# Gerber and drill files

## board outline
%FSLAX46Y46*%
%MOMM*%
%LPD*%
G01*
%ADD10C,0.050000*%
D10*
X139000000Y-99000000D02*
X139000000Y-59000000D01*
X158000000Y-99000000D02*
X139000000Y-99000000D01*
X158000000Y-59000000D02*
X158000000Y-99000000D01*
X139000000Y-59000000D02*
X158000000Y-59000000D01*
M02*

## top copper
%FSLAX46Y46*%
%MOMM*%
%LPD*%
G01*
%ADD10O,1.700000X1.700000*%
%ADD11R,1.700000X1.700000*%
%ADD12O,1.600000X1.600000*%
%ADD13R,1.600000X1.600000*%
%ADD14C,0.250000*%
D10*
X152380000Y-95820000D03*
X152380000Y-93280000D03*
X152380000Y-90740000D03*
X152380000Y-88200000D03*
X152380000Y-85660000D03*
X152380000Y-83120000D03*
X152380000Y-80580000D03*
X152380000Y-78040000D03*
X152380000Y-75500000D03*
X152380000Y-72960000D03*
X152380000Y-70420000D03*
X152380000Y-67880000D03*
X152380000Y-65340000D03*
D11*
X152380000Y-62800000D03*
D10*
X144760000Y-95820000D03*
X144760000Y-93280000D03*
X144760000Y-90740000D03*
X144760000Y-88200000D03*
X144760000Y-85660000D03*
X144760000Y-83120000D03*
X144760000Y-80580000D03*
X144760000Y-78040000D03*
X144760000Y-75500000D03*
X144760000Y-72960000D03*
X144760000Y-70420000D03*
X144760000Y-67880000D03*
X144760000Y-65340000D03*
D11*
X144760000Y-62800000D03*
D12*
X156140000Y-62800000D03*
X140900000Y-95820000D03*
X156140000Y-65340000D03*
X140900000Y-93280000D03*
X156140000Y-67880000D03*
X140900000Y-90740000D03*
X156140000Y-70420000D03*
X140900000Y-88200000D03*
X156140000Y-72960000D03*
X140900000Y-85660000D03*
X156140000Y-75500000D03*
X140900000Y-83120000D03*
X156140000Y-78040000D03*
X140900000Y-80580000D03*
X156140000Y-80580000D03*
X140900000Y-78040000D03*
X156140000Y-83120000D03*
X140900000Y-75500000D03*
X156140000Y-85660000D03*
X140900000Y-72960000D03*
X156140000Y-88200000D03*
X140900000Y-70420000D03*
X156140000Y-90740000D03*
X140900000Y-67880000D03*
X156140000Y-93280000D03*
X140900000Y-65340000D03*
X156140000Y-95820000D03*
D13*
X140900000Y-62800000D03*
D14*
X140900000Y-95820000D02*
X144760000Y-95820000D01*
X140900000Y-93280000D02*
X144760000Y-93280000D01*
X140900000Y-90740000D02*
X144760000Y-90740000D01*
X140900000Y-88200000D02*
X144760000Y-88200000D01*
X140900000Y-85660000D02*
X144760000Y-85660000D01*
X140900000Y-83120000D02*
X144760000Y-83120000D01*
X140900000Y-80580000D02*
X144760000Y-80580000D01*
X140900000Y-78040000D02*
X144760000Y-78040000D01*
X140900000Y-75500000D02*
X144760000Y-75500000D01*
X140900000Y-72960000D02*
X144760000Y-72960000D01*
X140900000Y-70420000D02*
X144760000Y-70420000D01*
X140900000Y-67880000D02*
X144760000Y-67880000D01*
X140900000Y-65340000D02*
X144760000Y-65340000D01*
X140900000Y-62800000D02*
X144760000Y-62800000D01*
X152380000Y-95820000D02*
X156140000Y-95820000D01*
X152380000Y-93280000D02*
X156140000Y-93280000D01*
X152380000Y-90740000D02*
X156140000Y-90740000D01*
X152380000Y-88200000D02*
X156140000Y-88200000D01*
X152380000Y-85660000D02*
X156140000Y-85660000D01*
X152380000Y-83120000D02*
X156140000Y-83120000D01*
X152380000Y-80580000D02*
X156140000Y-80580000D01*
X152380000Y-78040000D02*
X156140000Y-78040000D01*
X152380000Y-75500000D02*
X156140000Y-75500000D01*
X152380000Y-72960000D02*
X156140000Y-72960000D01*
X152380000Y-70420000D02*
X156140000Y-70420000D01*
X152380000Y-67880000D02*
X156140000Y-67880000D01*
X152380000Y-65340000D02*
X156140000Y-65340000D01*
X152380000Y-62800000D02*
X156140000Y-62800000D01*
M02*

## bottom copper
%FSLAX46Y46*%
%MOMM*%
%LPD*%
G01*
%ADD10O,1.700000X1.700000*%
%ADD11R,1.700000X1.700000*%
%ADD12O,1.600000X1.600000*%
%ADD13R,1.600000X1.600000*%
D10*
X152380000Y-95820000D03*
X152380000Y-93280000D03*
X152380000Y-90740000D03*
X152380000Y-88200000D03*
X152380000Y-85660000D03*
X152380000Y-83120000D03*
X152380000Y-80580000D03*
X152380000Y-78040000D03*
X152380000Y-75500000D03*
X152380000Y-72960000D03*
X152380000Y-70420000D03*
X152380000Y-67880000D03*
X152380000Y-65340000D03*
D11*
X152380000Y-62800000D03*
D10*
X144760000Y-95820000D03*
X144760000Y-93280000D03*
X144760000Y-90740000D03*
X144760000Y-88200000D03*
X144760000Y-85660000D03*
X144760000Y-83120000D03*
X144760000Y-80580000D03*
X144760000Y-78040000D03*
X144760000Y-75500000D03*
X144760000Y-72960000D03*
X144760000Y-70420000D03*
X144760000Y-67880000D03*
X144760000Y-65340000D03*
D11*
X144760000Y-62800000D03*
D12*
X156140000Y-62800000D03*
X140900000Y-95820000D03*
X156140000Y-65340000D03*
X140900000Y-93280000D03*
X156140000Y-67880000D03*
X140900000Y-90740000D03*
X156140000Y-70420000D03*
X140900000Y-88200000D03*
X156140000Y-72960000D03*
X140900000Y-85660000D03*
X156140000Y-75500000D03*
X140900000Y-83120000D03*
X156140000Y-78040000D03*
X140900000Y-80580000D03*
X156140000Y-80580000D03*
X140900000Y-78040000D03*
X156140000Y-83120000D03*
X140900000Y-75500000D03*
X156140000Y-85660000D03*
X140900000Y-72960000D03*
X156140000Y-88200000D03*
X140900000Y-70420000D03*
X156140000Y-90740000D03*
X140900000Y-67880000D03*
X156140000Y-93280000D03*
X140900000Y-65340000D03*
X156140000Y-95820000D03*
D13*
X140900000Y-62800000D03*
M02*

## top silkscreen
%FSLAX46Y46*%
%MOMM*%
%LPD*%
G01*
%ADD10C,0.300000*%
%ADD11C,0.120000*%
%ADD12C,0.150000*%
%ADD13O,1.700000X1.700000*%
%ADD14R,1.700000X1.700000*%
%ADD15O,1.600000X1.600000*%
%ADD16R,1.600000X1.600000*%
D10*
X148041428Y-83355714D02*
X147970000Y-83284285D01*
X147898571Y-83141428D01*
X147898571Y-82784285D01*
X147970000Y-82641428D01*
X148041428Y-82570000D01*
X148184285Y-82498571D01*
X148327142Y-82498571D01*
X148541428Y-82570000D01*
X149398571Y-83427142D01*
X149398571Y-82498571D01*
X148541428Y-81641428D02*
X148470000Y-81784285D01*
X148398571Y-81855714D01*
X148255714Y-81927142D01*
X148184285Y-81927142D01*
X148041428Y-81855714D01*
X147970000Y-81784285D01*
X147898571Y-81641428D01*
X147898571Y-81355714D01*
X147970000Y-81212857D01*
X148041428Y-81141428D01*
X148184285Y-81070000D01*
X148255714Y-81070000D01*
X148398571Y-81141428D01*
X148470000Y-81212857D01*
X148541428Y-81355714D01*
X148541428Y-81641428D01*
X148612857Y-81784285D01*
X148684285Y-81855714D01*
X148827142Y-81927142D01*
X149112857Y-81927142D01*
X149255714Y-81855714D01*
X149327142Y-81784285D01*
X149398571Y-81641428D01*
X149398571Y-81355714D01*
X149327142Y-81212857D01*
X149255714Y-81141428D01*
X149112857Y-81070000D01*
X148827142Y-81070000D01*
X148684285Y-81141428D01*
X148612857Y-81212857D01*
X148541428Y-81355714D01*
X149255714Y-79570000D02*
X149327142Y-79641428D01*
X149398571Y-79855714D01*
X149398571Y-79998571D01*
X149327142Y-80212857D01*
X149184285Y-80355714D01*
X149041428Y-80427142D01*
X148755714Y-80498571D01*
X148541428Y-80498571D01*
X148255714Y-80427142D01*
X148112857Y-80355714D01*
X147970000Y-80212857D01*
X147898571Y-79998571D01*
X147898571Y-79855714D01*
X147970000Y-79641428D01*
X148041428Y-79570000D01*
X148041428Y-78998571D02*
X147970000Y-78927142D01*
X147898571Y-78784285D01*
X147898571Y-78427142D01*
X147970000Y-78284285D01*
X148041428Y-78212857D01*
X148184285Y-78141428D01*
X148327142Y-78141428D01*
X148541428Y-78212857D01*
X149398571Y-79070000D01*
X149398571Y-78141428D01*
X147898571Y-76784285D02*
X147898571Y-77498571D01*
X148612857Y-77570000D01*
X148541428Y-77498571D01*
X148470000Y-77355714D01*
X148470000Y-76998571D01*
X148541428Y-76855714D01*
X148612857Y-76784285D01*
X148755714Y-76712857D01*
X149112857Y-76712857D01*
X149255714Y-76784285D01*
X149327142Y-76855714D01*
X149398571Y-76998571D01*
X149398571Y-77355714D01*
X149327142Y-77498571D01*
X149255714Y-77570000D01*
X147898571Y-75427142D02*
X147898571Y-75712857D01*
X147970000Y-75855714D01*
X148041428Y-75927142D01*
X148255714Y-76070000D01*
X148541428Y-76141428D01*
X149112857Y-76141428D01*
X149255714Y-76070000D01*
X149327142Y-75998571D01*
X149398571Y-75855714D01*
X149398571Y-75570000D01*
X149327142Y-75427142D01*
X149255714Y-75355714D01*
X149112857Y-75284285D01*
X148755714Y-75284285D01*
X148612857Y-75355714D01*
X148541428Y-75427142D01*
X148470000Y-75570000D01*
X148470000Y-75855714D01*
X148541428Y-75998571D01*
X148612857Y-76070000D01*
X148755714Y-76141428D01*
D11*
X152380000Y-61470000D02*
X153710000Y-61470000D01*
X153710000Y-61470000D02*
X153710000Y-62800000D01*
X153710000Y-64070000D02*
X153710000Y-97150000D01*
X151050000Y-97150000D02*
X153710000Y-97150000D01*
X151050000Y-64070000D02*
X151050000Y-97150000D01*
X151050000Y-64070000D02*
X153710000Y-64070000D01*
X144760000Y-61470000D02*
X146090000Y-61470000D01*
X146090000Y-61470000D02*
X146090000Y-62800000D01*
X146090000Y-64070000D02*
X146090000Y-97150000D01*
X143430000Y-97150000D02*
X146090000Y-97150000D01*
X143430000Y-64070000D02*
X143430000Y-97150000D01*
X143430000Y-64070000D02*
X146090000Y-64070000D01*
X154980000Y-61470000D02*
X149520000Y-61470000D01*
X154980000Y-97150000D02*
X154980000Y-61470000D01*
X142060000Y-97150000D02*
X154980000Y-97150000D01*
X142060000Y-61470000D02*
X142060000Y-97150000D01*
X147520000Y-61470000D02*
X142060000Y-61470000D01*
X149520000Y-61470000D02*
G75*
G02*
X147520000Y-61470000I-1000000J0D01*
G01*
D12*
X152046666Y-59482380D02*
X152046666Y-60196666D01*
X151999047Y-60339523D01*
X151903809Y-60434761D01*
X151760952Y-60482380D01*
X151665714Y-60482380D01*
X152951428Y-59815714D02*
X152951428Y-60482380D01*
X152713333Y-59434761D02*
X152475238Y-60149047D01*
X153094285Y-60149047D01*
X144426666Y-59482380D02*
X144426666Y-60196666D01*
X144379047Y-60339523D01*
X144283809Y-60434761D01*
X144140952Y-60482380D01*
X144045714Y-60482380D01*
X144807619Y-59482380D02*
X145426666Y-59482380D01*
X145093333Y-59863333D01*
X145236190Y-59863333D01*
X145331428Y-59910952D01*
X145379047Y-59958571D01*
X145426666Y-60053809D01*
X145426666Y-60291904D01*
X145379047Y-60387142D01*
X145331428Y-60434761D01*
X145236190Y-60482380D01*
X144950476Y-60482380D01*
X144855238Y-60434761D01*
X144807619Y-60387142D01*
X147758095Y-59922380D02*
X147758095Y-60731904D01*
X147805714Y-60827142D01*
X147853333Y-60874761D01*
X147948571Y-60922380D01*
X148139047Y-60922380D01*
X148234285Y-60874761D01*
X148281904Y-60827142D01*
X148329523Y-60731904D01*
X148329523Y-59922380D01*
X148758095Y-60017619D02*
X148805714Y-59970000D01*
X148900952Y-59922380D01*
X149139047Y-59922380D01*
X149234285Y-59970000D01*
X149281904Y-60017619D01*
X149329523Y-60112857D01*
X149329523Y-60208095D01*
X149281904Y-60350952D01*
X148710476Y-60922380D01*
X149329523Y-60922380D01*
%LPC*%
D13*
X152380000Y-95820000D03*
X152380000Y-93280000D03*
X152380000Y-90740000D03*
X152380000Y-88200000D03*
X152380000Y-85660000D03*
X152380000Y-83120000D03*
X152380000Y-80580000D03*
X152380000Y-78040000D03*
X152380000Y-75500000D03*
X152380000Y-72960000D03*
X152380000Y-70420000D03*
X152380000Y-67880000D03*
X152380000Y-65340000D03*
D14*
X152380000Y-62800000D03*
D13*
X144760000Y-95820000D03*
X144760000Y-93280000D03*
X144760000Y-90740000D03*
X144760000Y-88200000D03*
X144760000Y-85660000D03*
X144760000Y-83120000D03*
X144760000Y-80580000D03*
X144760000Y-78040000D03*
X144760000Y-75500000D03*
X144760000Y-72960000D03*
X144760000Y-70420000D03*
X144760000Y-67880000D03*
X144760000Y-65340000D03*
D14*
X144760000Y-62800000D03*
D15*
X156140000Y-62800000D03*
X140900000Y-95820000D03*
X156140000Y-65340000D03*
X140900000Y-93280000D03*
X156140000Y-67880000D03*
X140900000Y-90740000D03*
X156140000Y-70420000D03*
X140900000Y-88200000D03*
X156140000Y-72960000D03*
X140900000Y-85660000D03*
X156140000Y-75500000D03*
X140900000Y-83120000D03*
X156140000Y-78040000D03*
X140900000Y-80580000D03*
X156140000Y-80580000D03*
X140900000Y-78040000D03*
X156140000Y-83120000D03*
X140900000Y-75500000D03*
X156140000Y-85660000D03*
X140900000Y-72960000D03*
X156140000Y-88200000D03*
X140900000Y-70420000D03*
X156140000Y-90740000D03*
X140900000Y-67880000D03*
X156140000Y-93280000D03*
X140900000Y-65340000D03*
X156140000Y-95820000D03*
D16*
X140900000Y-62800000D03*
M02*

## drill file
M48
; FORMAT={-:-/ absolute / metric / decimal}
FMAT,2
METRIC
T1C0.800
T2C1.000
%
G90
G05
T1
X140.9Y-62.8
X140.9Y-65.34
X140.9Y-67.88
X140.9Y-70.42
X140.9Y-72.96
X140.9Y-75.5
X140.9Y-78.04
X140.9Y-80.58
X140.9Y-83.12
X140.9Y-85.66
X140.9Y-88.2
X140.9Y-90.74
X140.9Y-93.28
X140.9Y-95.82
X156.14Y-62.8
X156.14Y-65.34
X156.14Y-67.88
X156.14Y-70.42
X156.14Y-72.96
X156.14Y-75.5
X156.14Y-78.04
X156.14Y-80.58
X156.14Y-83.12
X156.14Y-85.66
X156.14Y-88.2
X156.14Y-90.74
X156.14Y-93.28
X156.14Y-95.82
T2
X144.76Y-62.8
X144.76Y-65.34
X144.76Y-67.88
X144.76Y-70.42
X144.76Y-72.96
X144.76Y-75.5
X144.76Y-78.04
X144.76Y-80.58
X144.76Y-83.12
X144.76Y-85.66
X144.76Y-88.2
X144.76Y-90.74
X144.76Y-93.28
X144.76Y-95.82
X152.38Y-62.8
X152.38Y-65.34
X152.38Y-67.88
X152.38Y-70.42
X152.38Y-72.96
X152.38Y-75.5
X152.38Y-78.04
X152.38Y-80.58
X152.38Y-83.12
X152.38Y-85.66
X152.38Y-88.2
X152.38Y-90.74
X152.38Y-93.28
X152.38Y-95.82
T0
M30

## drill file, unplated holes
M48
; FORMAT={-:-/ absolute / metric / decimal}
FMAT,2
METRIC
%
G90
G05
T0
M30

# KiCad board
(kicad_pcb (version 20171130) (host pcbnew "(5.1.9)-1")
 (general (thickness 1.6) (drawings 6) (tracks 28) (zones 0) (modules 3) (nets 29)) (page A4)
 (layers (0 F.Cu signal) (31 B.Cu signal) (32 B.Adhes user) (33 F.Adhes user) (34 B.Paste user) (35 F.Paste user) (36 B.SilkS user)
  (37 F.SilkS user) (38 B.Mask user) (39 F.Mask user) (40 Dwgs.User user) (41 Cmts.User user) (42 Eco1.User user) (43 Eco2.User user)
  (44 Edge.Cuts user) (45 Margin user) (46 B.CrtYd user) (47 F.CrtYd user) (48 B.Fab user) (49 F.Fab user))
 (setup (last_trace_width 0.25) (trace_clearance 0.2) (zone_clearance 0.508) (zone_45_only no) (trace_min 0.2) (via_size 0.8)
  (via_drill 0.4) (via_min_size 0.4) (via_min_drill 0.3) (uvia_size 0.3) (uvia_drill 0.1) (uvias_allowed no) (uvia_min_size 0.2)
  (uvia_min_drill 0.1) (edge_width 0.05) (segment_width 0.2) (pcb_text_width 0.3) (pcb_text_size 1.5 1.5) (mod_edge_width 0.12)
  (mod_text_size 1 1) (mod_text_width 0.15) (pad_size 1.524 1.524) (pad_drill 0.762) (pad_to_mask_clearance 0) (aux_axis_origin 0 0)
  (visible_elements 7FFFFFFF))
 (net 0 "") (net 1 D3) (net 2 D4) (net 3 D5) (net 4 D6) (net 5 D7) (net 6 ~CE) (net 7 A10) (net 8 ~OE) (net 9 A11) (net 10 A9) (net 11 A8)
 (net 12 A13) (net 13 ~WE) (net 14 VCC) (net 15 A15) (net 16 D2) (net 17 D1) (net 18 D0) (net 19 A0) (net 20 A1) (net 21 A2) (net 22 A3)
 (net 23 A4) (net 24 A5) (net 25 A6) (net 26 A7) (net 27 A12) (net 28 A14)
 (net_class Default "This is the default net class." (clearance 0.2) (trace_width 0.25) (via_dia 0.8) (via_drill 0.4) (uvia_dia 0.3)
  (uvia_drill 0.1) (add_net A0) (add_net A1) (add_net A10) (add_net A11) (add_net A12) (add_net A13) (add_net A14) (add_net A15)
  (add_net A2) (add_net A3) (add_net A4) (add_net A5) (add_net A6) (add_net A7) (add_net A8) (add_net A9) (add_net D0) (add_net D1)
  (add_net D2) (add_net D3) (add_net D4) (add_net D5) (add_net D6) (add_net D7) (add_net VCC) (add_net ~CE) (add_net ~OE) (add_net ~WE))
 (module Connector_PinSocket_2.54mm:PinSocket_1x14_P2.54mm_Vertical (layer F.Cu) (at 152.38 62.8)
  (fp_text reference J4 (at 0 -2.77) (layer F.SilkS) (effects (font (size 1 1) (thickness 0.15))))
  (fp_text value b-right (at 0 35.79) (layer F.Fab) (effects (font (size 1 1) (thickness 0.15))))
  (fp_line (start 0 -1.33) (end 1.33 -1.33) (layer F.SilkS) (width 0.12))
  (fp_line (start 1.33 -1.33) (end 1.33 0) (layer F.SilkS) (width 0.12))
  (fp_line (start 1.33 1.27) (end 1.33 34.35) (layer F.SilkS) (width 0.12))
  (fp_line (start -1.33 34.35) (end 1.33 34.35) (layer F.SilkS) (width 0.12))
  (fp_line (start -1.33 1.27) (end -1.33 34.35) (layer F.SilkS) (width 0.12))
  (fp_line (start -1.33 1.27) (end 1.33 1.27) (layer F.SilkS) (width 0.12))
  (pad 14 thru_hole oval (at 0 33.02) (size 1.7 1.7) (drill 1) (layers *.Cu *.Mask) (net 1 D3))
  (pad 13 thru_hole oval (at 0 30.48) (size 1.7 1.7) (drill 1) (layers *.Cu *.Mask) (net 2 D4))
  (pad 12 thru_hole oval (at 0 27.94) (size 1.7 1.7) (drill 1) (layers *.Cu *.Mask) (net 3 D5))
  (pad 11 thru_hole oval (at 0 25.4) (size 1.7 1.7) (drill 1) (layers *.Cu *.Mask) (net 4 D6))
  (pad 10 thru_hole oval (at 0 22.86) (size 1.7 1.7) (drill 1) (layers *.Cu *.Mask) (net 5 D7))
  (pad 9 thru_hole oval (at 0 20.32) (size 1.7 1.7) (drill 1) (layers *.Cu *.Mask) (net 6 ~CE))
  (pad 8 thru_hole oval (at 0 17.78) (size 1.7 1.7) (drill 1) (layers *.Cu *.Mask) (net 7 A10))
  (pad 7 thru_hole oval (at 0 15.24) (size 1.7 1.7) (drill 1) (layers *.Cu *.Mask) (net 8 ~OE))
  (pad 6 thru_hole oval (at 0 12.7) (size 1.7 1.7) (drill 1) (layers *.Cu *.Mask) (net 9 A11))
  (pad 5 thru_hole oval (at 0 10.16) (size 1.7 1.7) (drill 1) (layers *.Cu *.Mask) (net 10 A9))
  (pad 4 thru_hole oval (at 0 7.62) (size 1.7 1.7) (drill 1) (layers *.Cu *.Mask) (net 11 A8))
  (pad 3 thru_hole oval (at 0 5.08) (size 1.7 1.7) (drill 1) (layers *.Cu *.Mask) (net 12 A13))
  (pad 2 thru_hole oval (at 0 2.54) (size 1.7 1.7) (drill 1) (layers *.Cu *.Mask) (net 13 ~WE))
  (pad 1 thru_hole rect (at 0 0) (size 1.7 1.7) (drill 1) (layers *.Cu *.Mask) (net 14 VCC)))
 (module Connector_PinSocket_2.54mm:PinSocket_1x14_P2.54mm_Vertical (layer F.Cu) (at 144.76 62.8)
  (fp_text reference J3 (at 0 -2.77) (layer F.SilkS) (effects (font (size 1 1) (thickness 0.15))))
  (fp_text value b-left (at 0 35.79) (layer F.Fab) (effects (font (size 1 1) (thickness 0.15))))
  (fp_line (start 0 -1.33) (end 1.33 -1.33) (layer F.SilkS) (width 0.12))
  (fp_line (start 1.33 -1.33) (end 1.33 0) (layer F.SilkS) (width 0.12))
  (fp_line (start 1.33 1.27) (end 1.33 34.35) (layer F.SilkS) (width 0.12))
  (fp_line (start -1.33 34.35) (end 1.33 34.35) (layer F.SilkS) (width 0.12))
  (fp_line (start -1.33 1.27) (end -1.33 34.35) (layer F.SilkS) (width 0.12))
  (fp_line (start -1.33 1.27) (end 1.33 1.27) (layer F.SilkS) (width 0.12))
  (pad 14 thru_hole oval (at 0 33.02) (size 1.7 1.7) (drill 1) (layers *.Cu *.Mask) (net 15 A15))
  (pad 13 thru_hole oval (at 0 30.48) (size 1.7 1.7) (drill 1) (layers *.Cu *.Mask) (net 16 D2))
  (pad 12 thru_hole oval (at 0 27.94) (size 1.7 1.7) (drill 1) (layers *.Cu *.Mask) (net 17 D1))
  (pad 11 thru_hole oval (at 0 25.4) (size 1.7 1.7) (drill 1) (layers *.Cu *.Mask) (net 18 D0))
  (pad 10 thru_hole oval (at 0 22.86) (size 1.7 1.7) (drill 1) (layers *.Cu *.Mask) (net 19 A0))
  (pad 9 thru_hole oval (at 0 20.32) (size 1.7 1.7) (drill 1) (layers *.Cu *.Mask) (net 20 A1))
  (pad 8 thru_hole oval (at 0 17.78) (size 1.7 1.7) (drill 1) (layers *.Cu *.Mask) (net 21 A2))
  (pad 7 thru_hole oval (at 0 15.24) (size 1.7 1.7) (drill 1) (layers *.Cu *.Mask) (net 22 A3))
  (pad 6 thru_hole oval (at 0 12.7) (size 1.7 1.7) (drill 1) (layers *.Cu *.Mask) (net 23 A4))
  (pad 5 thru_hole oval (at 0 10.16) (size 1.7 1.7) (drill 1) (layers *.Cu *.Mask) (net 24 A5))
  (pad 4 thru_hole oval (at 0 7.62) (size 1.7 1.7) (drill 1) (layers *.Cu *.Mask) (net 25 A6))
  (pad 3 thru_hole oval (at 0 5.08) (size 1.7 1.7) (drill 1) (layers *.Cu *.Mask) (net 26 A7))
  (pad 2 thru_hole oval (at 0 2.54) (size 1.7 1.7) (drill 1) (layers *.Cu *.Mask) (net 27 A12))
  (pad 1 thru_hole rect (at 0 0) (size 1.7 1.7) (drill 1) (layers *.Cu *.Mask) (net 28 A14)))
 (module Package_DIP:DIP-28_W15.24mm (layer F.Cu) (at 140.9 62.8)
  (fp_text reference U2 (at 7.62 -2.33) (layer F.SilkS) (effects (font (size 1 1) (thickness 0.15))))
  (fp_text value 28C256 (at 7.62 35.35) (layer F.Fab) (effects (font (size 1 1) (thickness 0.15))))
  (fp_line (start 14.08 -1.33) (end 8.62 -1.33) (layer F.SilkS) (width 0.12))
  (fp_line (start 14.08 34.35) (end 14.08 -1.33) (layer F.SilkS) (width 0.12))
  (fp_line (start 1.16 34.35) (end 14.08 34.35) (layer F.SilkS) (width 0.12))
  (fp_line (start 1.16 -1.33) (end 1.16 34.35) (layer F.SilkS) (width 0.12))
  (fp_line (start 6.62 -1.33) (end 1.16 -1.33) (layer F.SilkS) (width 0.12))
  (fp_arc (start 7.62 -1.33) (end 6.62 -1.33) (angle -180) (layer F.SilkS) (width 0.12))
  (pad 28 thru_hole oval (at 15.24 0) (size 1.6 1.6) (drill 0.8) (layers *.Cu *.Mask) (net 14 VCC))
  (pad 14 thru_hole oval (at 0 33.02) (size 1.6 1.6) (drill 0.8) (layers *.Cu *.Mask) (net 15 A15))
  (pad 27 thru_hole oval (at 15.24 2.54) (size 1.6 1.6) (drill 0.8) (layers *.Cu *.Mask) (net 13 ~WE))
  (pad 13 thru_hole oval (at 0 30.48) (size 1.6 1.6) (drill 0.8) (layers *.Cu *.Mask) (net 16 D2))
  (pad 26 thru_hole oval (at 15.24 5.08) (size 1.6 1.6) (drill 0.8) (layers *.Cu *.Mask) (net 12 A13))
  (pad 12 thru_hole oval (at 0 27.94) (size 1.6 1.6) (drill 0.8) (layers *.Cu *.Mask) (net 17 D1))
  (pad 25 thru_hole oval (at 15.24 7.62) (size 1.6 1.6) (drill 0.8) (layers *.Cu *.Mask) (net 11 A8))
  (pad 11 thru_hole oval (at 0 25.4) (size 1.6 1.6) (drill 0.8) (layers *.Cu *.Mask) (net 18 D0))
  (pad 24 thru_hole oval (at 15.24 10.16) (size 1.6 1.6) (drill 0.8) (layers *.Cu *.Mask) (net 10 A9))
  (pad 10 thru_hole oval (at 0 22.86) (size 1.6 1.6) (drill 0.8) (layers *.Cu *.Mask) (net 19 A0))
  (pad 23 thru_hole oval (at 15.24 12.7) (size 1.6 1.6) (drill 0.8) (layers *.Cu *.Mask) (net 9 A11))
  (pad 9 thru_hole oval (at 0 20.32) (size 1.6 1.6) (drill 0.8) (layers *.Cu *.Mask) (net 20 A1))
  (pad 22 thru_hole oval (at 15.24 15.24) (size 1.6 1.6) (drill 0.8) (layers *.Cu *.Mask) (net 8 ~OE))
  (pad 8 thru_hole oval (at 0 17.78) (size 1.6 1.6) (drill 0.8) (layers *.Cu *.Mask) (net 21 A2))
  (pad 21 thru_hole oval (at 15.24 17.78) (size 1.6 1.6) (drill 0.8) (layers *.Cu *.Mask) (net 7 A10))
  (pad 7 thru_hole oval (at 0 15.24) (size 1.6 1.6) (drill 0.8) (layers *.Cu *.Mask) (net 22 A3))
  (pad 20 thru_hole oval (at 15.24 20.32) (size 1.6 1.6) (drill 0.8) (layers *.Cu *.Mask) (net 6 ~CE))
  (pad 6 thru_hole oval (at 0 12.7) (size 1.6 1.6) (drill 0.8) (layers *.Cu *.Mask) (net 23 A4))
  (pad 19 thru_hole oval (at 15.24 22.86) (size 1.6 1.6) (drill 0.8) (layers *.Cu *.Mask) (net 5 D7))
  (pad 5 thru_hole oval (at 0 10.16) (size 1.6 1.6) (drill 0.8) (layers *.Cu *.Mask) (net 24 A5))
  (pad 18 thru_hole oval (at 15.24 25.4) (size 1.6 1.6) (drill 0.8) (layers *.Cu *.Mask) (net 4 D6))
  (pad 4 thru_hole oval (at 0 7.62) (size 1.6 1.6) (drill 0.8) (layers *.Cu *.Mask) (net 25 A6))
  (pad 17 thru_hole oval (at 15.24 27.94) (size 1.6 1.6) (drill 0.8) (layers *.Cu *.Mask) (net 3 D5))
  (pad 3 thru_hole oval (at 0 5.08) (size 1.6 1.6) (drill 0.8) (layers *.Cu *.Mask) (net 26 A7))
  (pad 16 thru_hole oval (at 15.24 30.48) (size 1.6 1.6) (drill 0.8) (layers *.Cu *.Mask) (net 2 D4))
  (pad 2 thru_hole oval (at 0 2.54) (size 1.6 1.6) (drill 0.8) (layers *.Cu *.Mask) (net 27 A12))
  (pad 15 thru_hole oval (at 15.24 33.02) (size 1.6 1.6) (drill 0.8) (layers *.Cu *.Mask) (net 1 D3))
  (pad 1 thru_hole rect (at 0 0) (size 1.6 1.6) (drill 0.8) (layers *.Cu *.Mask) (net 28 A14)))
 (gr_line (start 139 99) (end 139 59) (layer Edge.Cuts) (width 0.05))
 (gr_line (start 158 99) (end 139 99) (layer Edge.Cuts) (width 0.05))
 (gr_line (start 158 59) (end 158 99) (layer Edge.Cuts) (width 0.05))
 (gr_line (start 139 59) (end 158 59) (layer Edge.Cuts) (width 0.05))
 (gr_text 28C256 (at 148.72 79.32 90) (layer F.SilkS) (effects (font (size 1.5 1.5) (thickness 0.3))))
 (segment (start 140.9 95.82) (end 144.76 95.82) (width 0.25) (layer F.Cu) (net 15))
 (segment (start 140.9 93.28) (end 144.76 93.28) (width 0.25) (layer F.Cu) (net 16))
 (segment (start 140.9 90.74) (end 144.76 90.74) (width 0.25) (layer F.Cu) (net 17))
 (segment (start 140.9 88.2) (end 144.76 88.2) (width 0.25) (layer F.Cu) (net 18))
 (segment (start 140.9 85.66) (end 144.76 85.66) (width 0.25) (layer F.Cu) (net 19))
 (segment (start 140.9 83.12) (end 144.76 83.12) (width 0.25) (layer F.Cu) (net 20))
 (segment (start 140.9 80.58) (end 144.76 80.58) (width 0.25) (layer F.Cu) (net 21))
 (segment (start 140.9 78.04) (end 144.76 78.04) (width 0.25) (layer F.Cu) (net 22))
 (segment (start 140.9 75.5) (end 144.76 75.5) (width 0.25) (layer F.Cu) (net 23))
 (segment (start 140.9 72.96) (end 144.76 72.96) (width 0.25) (layer F.Cu) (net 24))
 (segment (start 140.9 70.42) (end 144.76 70.42) (width 0.25) (layer F.Cu) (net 25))
 (segment (start 140.9 67.88) (end 144.76 67.88) (width 0.25) (layer F.Cu) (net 26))
 (segment (start 140.9 65.34) (end 144.76 65.34) (width 0.25) (layer F.Cu) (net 27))
 (segment (start 140.9 62.8) (end 144.76 62.8) (width 0.25) (layer F.Cu) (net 28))
 (segment (start 152.38 95.82) (end 156.14 95.82) (width 0.25) (layer F.Cu) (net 1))
 (segment (start 152.38 93.28) (end 156.14 93.28) (width 0.25) (layer F.Cu) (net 2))
 (segment (start 152.38 90.74) (end 156.14 90.74) (width 0.25) (layer F.Cu) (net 3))
 (segment (start 152.38 88.2) (end 156.14 88.2) (width 0.25) (layer F.Cu) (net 4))
 (segment (start 152.38 85.66) (end 156.14 85.66) (width 0.25) (layer F.Cu) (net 5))
 (segment (start 152.38 83.12) (end 156.14 83.12) (width 0.25) (layer F.Cu) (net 6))
 (segment (start 152.38 80.58) (end 156.14 80.58) (width 0.25) (layer F.Cu) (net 7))
 (segment (start 152.38 78.04) (end 156.14 78.04) (width 0.25) (layer F.Cu) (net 8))
 (segment (start 152.38 75.5) (end 156.14 75.5) (width 0.25) (layer F.Cu) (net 9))
 (segment (start 152.38 72.96) (end 156.14 72.96) (width 0.25) (layer F.Cu) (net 10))
 (segment (start 152.38 70.42) (end 156.14 70.42) (width 0.25) (layer F.Cu) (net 11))
 (segment (start 152.38 67.88) (end 156.14 67.88) (width 0.25) (layer F.Cu) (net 12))
 (segment (start 152.38 65.34) (end 156.14 65.34) (width 0.25) (layer F.Cu) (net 13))
 (segment (start 152.38 62.8) (end 156.14 62.8) (width 0.25) (layer F.Cu) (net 14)))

